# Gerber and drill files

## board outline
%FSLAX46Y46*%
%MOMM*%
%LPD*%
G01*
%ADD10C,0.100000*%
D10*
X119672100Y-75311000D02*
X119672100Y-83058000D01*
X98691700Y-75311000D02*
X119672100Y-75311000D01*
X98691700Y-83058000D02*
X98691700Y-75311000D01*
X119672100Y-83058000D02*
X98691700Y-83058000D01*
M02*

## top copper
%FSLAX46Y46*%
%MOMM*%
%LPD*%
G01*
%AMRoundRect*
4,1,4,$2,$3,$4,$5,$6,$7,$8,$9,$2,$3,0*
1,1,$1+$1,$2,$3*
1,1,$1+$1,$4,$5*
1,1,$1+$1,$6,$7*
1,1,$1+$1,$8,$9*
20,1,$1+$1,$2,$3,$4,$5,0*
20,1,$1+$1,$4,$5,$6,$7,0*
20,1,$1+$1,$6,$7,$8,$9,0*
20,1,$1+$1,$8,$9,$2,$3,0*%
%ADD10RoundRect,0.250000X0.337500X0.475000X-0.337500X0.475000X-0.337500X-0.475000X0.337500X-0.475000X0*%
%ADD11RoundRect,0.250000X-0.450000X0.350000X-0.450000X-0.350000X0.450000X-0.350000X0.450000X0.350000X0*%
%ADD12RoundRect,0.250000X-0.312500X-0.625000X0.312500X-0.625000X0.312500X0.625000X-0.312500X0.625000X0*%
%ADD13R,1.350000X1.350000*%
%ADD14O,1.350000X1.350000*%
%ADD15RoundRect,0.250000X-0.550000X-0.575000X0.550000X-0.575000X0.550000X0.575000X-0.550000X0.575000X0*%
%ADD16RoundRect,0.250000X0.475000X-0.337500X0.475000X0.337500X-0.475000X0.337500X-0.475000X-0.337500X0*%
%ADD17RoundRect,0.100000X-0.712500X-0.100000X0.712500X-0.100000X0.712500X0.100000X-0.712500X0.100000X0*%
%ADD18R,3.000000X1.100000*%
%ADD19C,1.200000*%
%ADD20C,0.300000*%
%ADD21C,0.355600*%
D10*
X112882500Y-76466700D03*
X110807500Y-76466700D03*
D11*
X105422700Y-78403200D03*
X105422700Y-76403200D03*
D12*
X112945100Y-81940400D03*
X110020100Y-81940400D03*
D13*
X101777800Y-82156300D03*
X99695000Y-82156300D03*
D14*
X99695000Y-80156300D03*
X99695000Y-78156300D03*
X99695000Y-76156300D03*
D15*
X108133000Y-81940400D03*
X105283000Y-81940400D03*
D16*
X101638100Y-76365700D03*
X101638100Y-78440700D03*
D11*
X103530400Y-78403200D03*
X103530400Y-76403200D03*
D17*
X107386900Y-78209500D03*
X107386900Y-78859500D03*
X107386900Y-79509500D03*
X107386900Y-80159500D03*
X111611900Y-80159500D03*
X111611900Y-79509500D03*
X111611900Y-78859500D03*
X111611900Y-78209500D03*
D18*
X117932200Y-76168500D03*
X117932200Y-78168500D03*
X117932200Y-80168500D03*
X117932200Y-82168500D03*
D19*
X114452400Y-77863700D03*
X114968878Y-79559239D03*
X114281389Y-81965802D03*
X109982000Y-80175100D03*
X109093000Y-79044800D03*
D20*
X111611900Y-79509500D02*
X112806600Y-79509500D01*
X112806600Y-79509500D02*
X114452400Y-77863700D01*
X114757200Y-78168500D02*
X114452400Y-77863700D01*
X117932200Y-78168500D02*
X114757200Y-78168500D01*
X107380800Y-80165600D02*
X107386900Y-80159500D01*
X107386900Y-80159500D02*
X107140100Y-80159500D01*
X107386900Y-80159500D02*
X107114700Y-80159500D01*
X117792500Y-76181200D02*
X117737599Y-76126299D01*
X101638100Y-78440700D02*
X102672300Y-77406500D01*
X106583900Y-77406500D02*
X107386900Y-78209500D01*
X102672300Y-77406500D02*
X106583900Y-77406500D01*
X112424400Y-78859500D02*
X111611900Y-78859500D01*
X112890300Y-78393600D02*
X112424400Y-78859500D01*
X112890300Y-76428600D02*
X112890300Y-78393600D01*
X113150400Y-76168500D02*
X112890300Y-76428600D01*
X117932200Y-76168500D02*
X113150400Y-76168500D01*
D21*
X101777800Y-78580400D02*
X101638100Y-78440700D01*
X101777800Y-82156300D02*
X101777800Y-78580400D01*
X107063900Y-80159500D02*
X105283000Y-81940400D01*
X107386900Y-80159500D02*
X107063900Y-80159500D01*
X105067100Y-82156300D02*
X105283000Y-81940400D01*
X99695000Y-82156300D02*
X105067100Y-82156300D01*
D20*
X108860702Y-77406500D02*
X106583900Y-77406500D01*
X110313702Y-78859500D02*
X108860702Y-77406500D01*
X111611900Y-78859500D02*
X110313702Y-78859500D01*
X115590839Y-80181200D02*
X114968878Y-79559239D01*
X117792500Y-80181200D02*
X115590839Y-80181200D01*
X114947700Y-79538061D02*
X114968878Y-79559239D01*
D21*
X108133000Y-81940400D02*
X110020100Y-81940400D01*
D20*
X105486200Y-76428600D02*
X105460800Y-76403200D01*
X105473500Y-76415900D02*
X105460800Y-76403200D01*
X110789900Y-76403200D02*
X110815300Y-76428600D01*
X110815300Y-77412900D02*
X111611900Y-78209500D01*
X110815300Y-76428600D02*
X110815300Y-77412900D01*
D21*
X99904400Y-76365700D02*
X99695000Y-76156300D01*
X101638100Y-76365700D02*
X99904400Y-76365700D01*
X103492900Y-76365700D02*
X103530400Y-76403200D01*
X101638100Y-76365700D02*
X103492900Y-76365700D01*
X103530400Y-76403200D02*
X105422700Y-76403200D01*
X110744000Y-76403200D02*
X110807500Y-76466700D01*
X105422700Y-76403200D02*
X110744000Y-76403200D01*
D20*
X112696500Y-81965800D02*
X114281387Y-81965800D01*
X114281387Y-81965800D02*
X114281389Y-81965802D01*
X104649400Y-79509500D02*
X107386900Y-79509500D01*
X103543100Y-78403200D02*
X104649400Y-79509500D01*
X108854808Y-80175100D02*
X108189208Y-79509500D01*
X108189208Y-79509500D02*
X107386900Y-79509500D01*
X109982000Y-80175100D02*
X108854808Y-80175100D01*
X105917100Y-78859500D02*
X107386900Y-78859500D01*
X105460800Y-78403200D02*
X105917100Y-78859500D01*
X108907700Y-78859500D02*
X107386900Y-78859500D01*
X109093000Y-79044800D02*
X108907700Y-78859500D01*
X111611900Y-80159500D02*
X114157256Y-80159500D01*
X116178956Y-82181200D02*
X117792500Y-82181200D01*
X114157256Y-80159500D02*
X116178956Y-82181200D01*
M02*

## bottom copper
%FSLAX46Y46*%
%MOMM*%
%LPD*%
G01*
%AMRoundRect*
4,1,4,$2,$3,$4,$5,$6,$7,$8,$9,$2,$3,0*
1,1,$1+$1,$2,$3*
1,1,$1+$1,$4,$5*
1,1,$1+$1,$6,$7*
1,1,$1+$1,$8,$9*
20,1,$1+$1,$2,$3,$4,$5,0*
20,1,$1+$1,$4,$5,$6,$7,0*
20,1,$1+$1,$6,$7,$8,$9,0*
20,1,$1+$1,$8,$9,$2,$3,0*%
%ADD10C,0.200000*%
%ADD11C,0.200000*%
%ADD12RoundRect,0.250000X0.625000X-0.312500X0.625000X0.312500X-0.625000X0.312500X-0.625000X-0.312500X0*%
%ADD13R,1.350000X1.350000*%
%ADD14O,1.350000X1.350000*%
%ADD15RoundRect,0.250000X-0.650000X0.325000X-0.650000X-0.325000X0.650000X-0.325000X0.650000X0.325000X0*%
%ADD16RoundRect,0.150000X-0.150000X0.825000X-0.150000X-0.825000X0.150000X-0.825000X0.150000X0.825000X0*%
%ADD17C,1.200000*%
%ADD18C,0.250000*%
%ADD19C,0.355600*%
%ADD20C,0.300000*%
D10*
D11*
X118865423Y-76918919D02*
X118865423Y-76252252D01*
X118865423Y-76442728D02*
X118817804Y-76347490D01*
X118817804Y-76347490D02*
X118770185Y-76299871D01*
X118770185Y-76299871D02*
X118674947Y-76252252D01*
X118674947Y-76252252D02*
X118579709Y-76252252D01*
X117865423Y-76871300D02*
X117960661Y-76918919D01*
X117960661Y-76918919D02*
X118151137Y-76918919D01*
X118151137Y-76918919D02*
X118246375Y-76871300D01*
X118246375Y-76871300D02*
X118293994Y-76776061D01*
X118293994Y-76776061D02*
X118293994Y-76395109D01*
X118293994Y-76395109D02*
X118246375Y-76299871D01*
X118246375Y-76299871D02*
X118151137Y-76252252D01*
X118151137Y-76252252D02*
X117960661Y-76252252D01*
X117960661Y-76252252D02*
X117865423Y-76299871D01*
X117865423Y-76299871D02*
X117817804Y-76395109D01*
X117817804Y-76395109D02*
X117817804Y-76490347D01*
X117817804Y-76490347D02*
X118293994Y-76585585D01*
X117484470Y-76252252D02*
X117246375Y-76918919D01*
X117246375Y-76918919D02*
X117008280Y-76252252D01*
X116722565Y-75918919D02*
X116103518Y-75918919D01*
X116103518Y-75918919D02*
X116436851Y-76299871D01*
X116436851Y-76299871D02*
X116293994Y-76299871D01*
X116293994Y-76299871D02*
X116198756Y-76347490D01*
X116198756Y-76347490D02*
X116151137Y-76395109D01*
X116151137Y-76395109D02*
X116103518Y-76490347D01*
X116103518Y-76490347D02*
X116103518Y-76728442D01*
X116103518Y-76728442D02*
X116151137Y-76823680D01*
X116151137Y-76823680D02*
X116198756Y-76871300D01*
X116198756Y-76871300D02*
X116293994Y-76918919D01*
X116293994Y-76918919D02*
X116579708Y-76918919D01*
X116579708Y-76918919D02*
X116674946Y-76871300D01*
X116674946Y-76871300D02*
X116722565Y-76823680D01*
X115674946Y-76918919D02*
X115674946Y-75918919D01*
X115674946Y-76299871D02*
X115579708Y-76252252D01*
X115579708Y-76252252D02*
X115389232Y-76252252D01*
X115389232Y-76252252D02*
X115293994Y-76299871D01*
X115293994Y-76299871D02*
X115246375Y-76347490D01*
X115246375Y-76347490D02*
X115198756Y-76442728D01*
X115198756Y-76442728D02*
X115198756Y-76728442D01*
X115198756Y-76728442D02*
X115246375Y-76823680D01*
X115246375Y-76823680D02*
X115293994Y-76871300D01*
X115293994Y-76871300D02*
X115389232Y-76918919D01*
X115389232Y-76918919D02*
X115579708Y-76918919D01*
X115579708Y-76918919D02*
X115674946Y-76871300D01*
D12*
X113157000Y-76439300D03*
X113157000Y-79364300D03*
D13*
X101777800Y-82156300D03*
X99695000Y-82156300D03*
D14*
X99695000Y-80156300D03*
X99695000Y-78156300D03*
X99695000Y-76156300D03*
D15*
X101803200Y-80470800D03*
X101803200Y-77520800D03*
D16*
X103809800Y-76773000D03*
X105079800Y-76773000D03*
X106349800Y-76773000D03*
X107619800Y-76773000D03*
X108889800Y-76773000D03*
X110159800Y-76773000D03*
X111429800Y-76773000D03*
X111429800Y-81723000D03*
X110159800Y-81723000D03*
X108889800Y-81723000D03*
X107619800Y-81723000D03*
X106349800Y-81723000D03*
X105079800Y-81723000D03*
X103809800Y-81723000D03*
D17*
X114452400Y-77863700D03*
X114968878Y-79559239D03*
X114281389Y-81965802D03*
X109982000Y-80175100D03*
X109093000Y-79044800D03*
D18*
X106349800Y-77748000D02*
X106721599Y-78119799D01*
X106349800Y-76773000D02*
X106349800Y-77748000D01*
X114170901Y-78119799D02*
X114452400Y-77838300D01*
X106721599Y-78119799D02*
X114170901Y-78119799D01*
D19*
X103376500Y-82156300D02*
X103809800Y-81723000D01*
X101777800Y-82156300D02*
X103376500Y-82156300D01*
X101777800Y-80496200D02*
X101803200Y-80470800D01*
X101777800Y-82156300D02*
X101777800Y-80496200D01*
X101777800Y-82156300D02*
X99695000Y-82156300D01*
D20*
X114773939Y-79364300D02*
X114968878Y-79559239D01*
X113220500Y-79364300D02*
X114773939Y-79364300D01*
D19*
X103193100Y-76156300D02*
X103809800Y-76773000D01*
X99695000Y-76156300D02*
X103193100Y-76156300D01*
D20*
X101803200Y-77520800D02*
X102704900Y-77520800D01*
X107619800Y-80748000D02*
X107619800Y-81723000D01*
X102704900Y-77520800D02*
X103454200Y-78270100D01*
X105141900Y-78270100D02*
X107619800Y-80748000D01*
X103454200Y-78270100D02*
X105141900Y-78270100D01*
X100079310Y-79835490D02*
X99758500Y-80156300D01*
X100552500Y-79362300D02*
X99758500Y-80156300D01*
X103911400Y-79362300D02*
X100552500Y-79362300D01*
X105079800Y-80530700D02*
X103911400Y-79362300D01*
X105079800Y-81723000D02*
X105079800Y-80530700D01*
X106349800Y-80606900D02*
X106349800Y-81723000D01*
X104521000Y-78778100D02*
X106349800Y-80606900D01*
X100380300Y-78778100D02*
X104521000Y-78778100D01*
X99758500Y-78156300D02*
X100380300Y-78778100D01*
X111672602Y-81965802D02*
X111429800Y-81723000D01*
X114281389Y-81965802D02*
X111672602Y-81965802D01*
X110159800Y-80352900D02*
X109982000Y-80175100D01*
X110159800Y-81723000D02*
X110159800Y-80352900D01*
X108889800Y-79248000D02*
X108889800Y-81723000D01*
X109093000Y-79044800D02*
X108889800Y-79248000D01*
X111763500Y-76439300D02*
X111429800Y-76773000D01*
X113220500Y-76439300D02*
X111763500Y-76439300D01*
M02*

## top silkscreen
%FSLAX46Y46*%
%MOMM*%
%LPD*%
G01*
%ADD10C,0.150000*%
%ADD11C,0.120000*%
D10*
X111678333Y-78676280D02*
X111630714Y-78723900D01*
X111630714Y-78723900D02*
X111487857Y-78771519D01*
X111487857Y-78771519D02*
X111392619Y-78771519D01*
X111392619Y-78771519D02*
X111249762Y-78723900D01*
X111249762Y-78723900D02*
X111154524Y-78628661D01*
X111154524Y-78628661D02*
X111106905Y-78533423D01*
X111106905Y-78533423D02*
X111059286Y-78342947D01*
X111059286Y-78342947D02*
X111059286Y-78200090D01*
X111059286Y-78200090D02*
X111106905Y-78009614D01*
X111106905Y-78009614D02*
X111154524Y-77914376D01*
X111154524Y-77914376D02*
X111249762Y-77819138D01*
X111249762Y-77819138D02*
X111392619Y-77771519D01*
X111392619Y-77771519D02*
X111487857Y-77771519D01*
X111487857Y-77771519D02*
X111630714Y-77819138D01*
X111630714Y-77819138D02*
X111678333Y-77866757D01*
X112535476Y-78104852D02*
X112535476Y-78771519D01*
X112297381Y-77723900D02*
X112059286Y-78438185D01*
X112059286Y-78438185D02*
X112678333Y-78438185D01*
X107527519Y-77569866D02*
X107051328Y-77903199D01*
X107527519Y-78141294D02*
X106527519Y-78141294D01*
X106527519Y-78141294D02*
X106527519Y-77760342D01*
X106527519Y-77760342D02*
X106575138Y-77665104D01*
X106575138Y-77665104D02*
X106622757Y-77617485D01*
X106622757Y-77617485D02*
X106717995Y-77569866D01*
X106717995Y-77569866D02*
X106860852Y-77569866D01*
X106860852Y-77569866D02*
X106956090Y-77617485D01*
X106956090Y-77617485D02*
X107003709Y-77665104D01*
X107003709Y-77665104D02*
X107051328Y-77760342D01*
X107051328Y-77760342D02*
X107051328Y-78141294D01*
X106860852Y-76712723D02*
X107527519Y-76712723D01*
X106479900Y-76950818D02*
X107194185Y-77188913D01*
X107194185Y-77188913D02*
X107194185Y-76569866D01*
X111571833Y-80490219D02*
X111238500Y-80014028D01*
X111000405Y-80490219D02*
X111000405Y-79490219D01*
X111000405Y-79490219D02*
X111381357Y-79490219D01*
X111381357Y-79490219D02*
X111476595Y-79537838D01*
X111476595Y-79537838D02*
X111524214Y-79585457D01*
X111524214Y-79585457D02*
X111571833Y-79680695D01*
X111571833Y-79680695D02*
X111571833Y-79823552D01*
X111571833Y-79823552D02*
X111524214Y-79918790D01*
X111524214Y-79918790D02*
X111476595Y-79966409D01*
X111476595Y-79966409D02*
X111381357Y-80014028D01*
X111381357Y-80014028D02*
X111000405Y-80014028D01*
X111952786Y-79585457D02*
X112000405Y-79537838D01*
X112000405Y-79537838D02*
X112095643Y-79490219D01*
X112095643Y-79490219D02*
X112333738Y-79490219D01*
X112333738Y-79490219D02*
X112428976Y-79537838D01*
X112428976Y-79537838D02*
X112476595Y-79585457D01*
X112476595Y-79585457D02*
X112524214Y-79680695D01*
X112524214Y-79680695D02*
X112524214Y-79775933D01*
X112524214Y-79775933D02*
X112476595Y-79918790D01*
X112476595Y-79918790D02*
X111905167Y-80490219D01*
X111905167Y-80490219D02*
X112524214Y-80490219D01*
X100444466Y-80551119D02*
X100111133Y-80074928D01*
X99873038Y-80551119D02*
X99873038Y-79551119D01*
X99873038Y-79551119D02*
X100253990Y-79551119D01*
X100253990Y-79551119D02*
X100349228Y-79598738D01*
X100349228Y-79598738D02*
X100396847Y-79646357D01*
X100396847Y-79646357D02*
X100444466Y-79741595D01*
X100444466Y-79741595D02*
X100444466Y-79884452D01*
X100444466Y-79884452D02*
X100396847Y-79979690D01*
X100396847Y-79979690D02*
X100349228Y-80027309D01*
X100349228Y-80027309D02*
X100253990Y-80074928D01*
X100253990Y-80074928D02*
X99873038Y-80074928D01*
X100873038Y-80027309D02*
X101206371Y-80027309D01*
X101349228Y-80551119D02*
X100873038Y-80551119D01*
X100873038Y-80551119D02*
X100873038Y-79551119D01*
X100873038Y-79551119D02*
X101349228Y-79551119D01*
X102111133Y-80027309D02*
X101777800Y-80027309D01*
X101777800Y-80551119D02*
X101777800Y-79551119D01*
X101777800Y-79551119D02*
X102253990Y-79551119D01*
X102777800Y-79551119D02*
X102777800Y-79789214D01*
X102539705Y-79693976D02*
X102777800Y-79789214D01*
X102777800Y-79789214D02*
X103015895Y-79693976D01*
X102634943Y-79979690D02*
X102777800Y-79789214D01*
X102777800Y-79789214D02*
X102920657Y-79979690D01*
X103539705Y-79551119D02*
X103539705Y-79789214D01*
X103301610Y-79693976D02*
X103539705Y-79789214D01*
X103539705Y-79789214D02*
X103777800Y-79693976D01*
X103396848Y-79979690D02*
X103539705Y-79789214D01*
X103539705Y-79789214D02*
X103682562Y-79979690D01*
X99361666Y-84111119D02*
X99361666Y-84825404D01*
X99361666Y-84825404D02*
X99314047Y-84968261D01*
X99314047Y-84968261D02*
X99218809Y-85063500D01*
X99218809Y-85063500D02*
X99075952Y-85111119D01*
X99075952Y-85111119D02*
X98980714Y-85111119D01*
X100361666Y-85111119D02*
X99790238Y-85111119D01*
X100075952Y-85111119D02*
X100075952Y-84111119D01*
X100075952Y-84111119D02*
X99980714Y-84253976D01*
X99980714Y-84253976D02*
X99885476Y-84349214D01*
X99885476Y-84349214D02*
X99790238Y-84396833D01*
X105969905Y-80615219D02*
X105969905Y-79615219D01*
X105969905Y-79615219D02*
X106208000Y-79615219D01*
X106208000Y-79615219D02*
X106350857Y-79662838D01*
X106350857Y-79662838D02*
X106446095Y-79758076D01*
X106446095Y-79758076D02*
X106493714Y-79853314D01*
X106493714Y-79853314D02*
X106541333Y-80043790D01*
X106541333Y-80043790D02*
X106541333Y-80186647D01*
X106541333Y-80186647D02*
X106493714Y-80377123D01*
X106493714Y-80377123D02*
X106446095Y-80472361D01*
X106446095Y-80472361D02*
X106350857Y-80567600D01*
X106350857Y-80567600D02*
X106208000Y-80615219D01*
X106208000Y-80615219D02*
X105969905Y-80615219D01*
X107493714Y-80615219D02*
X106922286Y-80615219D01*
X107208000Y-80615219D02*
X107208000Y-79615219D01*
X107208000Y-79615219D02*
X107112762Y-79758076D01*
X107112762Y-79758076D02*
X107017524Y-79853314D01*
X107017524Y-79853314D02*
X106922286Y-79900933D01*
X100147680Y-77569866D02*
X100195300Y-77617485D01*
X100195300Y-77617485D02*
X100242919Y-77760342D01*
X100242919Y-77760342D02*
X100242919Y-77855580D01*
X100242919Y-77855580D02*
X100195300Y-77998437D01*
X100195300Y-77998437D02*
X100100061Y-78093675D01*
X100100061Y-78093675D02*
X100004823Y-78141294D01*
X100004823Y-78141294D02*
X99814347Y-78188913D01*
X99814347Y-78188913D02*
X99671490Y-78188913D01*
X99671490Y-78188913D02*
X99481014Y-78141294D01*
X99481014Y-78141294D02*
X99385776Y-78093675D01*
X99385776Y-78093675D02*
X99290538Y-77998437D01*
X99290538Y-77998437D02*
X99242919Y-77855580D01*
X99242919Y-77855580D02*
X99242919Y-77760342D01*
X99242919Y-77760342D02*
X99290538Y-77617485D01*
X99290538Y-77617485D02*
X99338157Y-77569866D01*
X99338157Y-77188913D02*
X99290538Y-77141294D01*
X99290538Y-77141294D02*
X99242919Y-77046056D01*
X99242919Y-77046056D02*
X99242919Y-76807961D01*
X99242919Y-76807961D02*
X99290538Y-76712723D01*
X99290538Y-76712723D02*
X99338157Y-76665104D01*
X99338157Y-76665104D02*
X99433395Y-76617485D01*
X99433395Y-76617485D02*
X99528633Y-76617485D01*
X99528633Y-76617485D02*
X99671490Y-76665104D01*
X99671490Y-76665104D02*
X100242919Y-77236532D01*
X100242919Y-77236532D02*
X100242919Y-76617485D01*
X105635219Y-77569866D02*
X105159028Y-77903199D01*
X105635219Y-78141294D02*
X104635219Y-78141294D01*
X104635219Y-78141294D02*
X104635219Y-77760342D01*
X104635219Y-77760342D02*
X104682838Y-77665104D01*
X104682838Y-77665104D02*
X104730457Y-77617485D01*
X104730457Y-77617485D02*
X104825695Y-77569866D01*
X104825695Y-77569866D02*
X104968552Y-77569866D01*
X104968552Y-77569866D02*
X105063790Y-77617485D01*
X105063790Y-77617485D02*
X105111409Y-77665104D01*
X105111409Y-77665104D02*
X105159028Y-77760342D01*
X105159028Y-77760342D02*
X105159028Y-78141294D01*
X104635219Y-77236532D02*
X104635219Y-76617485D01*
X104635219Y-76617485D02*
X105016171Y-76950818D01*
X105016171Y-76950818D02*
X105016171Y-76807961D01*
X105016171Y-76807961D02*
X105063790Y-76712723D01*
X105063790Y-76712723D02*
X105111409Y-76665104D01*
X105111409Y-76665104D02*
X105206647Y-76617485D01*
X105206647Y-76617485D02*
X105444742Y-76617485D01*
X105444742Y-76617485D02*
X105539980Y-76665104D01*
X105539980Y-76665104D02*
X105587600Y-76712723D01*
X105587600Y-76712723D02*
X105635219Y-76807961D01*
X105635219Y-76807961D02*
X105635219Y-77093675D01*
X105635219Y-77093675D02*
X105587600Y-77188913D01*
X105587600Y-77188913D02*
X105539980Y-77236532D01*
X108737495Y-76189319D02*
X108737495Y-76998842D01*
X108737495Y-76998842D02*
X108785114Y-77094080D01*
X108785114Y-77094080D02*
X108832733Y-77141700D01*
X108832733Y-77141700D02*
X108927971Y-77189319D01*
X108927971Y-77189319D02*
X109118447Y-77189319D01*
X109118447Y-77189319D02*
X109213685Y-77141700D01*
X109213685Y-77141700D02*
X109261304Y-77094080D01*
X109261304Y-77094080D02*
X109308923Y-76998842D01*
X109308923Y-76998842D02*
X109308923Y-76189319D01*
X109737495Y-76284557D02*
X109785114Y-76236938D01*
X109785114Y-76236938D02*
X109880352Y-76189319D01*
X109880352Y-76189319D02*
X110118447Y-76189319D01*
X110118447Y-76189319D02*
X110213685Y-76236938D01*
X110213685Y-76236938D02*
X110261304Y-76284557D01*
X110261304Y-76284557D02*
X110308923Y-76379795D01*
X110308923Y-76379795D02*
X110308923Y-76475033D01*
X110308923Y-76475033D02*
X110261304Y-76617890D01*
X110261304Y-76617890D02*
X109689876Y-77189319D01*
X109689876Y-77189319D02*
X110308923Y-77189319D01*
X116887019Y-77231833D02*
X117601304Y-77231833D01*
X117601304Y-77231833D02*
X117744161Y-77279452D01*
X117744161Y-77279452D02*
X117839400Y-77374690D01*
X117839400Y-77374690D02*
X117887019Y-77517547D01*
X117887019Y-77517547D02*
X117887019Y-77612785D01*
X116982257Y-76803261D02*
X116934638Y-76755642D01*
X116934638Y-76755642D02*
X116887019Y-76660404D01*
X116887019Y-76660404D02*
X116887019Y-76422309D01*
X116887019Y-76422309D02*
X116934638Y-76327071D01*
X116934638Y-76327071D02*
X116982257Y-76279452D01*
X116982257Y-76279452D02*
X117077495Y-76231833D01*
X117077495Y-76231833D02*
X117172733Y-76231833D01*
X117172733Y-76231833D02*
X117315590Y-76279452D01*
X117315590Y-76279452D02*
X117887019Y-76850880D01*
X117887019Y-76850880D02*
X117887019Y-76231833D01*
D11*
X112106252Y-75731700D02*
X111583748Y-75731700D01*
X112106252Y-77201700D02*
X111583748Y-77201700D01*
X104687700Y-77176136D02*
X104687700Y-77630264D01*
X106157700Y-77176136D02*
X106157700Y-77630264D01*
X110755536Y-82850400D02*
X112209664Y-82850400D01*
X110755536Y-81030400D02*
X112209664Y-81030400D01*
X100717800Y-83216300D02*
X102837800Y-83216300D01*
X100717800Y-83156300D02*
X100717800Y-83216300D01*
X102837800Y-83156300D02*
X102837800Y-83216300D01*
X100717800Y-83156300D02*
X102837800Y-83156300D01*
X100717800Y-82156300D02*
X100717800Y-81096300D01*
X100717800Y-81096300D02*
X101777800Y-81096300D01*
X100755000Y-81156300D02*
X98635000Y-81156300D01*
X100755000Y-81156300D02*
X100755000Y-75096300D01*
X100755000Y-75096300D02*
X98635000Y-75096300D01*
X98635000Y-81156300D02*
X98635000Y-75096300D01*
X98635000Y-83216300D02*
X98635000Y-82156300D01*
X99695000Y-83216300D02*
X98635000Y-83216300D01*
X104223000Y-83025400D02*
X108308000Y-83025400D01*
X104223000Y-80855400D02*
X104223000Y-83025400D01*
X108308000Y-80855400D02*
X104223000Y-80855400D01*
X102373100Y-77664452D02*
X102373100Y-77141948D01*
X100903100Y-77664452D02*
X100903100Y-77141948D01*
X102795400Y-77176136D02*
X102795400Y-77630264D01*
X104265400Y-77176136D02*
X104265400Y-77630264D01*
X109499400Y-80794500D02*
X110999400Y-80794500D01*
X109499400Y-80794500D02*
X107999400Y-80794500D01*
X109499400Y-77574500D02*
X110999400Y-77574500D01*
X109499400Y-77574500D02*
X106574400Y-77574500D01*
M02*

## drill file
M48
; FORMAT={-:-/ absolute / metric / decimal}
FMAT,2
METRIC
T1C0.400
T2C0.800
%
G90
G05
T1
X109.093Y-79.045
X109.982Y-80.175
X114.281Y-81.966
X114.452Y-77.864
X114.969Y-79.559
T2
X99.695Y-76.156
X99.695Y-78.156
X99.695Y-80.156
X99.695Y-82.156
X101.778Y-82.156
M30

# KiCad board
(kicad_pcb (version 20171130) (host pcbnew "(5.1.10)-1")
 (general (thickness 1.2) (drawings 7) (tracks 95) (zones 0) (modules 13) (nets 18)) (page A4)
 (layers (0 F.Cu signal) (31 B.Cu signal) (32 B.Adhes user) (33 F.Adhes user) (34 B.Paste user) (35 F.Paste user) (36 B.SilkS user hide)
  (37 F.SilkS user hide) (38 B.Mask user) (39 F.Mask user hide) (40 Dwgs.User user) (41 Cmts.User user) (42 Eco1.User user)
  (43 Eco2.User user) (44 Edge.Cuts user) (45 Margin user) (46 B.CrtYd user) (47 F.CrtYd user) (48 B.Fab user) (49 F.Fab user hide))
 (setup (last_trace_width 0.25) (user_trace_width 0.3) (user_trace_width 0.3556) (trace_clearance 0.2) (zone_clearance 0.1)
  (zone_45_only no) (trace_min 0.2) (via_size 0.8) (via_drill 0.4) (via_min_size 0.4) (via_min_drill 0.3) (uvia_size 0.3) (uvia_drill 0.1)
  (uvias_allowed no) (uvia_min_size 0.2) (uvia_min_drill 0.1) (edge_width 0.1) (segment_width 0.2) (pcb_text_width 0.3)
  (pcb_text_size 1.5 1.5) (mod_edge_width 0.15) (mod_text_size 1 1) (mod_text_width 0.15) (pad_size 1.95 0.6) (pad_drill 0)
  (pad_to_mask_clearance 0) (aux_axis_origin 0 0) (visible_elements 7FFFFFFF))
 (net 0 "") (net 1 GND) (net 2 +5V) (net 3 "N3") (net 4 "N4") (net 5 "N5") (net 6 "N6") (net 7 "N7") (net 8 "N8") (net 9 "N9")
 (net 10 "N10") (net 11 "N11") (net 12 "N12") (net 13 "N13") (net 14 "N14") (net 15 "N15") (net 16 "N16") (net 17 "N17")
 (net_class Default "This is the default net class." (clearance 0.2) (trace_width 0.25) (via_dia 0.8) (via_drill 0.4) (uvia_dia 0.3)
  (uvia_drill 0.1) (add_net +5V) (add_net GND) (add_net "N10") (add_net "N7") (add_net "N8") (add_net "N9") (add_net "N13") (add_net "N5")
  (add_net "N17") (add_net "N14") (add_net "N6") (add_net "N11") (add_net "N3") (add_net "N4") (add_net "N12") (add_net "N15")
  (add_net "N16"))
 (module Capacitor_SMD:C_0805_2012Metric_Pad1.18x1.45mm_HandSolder (layer F.Cu) (at 111.845 76.4667 180)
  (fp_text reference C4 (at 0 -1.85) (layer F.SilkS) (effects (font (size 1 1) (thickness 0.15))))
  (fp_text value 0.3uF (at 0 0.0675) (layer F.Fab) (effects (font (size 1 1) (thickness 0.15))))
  (fp_line (start -0.261252 0.735) (end 0.261252 0.735) (layer F.SilkS) (width 0.12))
  (fp_line (start -0.261252 -0.735) (end 0.261252 -0.735) (layer F.SilkS) (width 0.12))
  (pad 1 smd roundrect (at -1.0375 0 180) (size 1.175 1.45) (layers F.Cu F.Paste F.Mask) (roundrect_rratio 0.212766) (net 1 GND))
  (pad 2 smd roundrect (at 1.0375 0 180) (size 1.175 1.45) (layers F.Cu F.Paste F.Mask) (roundrect_rratio 0.212766) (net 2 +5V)))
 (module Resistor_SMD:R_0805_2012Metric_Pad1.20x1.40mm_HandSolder (layer F.Cu) (at 105.4227 77.4032 270)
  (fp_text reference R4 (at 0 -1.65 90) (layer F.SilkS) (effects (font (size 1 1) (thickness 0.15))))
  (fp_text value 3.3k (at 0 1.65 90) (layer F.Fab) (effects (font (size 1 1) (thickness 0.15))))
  (fp_line (start -0.227064 0.735) (end 0.227064 0.735) (layer F.SilkS) (width 0.12))
  (fp_line (start -0.227064 -0.735) (end 0.227064 -0.735) (layer F.SilkS) (width 0.12))
  (pad 2 smd roundrect (at 1 0 270) (size 1.2 1.4) (layers F.Cu F.Paste F.Mask) (roundrect_rratio 0.208333) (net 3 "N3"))
  (pad 1 smd roundrect (at -1 0 270) (size 1.2 1.4) (layers F.Cu F.Paste F.Mask) (roundrect_rratio 0.208333) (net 2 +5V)))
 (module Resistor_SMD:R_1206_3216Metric (layer B.Cu) (at 113.157 77.9018 90)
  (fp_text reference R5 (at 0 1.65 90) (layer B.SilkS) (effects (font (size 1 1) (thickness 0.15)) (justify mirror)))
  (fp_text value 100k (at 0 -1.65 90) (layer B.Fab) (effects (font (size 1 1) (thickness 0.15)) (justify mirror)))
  (pad 2 smd roundrect (at 1.4625 0 90) (size 1.125 1.75) (layers B.Cu B.Paste B.Mask) (roundrect_rratio 0.222222) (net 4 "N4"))
  (pad 1 smd roundrect (at -1.4625 0 90) (size 1.125 1.75) (layers B.Cu B.Paste B.Mask) (roundrect_rratio 0.222222) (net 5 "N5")))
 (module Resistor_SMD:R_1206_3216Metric (layer F.Cu) (at 111.4826 81.9404)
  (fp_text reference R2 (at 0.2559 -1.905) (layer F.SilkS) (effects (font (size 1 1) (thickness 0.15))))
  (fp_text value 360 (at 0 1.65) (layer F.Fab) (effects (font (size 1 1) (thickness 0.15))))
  (fp_line (start -0.727064 0.91) (end 0.727064 0.91) (layer F.SilkS) (width 0.12))
  (fp_line (start -0.727064 -0.91) (end 0.727064 -0.91) (layer F.SilkS) (width 0.12))
  (pad 2 smd roundrect (at 1.4625 0) (size 1.125 1.75) (layers F.Cu F.Paste F.Mask) (roundrect_rratio 0.222222) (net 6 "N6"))
  (pad 1 smd roundrect (at -1.4625 0) (size 1.125 1.75) (layers F.Cu F.Paste F.Mask) (roundrect_rratio 0.222222) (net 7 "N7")))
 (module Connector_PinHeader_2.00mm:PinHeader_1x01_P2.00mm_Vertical (layer F.Cu) (at 101.7778 82.1563)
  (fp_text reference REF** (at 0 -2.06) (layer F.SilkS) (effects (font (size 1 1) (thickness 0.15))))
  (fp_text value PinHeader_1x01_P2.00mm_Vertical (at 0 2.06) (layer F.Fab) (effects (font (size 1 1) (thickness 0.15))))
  (fp_line (start -1.06 1.06) (end 1.06 1.06) (layer F.SilkS) (width 0.12))
  (fp_line (start -1.06 1) (end -1.06 1.06) (layer F.SilkS) (width 0.12))
  (fp_line (start 1.06 1) (end 1.06 1.06) (layer F.SilkS) (width 0.12))
  (fp_line (start -1.06 1) (end 1.06 1) (layer F.SilkS) (width 0.12))
  (fp_line (start -1.06 0) (end -1.06 -1.06) (layer F.SilkS) (width 0.12))
  (fp_line (start -1.06 -1.06) (end 0 -1.06) (layer F.SilkS) (width 0.12))
  (pad 1 thru_hole rect (at 0 0) (size 1.35 1.35) (drill 0.8) (layers *.Cu *.Mask) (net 1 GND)))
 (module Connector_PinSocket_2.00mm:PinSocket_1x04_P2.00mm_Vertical (layer F.Cu) (at 99.695 82.1563 180)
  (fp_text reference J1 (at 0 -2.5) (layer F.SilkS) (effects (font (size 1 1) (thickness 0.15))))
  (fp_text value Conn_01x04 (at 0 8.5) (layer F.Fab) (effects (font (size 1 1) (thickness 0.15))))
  (fp_line (start -1.06 1) (end 1.06 1) (layer F.SilkS) (width 0.12))
  (fp_line (start -1.06 1) (end -1.06 7.06) (layer F.SilkS) (width 0.12))
  (fp_line (start -1.06 7.06) (end 1.06 7.06) (layer F.SilkS) (width 0.12))
  (fp_line (start 1.06 1) (end 1.06 7.06) (layer F.SilkS) (width 0.12))
  (fp_line (start 1.06 -1.06) (end 1.06 0) (layer F.SilkS) (width 0.12))
  (fp_line (start 0 -1.06) (end 1.06 -1.06) (layer F.SilkS) (width 0.12))
  (pad 1 thru_hole rect (at 0 0 180) (size 1.35 1.35) (drill 0.8) (layers *.Cu *.Mask) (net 1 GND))
  (pad 2 thru_hole oval (at 0 2 180) (size 1.35 1.35) (drill 0.8) (layers *.Cu *.Mask) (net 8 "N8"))
  (pad 3 thru_hole oval (at 0 4 180) (size 1.35 1.35) (drill 0.8) (layers *.Cu *.Mask) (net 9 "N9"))
  (pad 4 thru_hole oval (at 0 6 180) (size 1.35 1.35) (drill 0.8) (layers *.Cu *.Mask) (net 2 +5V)))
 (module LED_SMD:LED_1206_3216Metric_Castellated (layer F.Cu) (at 106.708 81.9404)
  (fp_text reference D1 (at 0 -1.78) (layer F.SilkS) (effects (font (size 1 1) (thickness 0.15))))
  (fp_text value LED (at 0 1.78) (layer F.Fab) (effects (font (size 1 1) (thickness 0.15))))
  (fp_line (start -2.485 1.085) (end 1.6 1.085) (layer F.SilkS) (width 0.12))
  (fp_line (start -2.485 -1.085) (end -2.485 1.085) (layer F.SilkS) (width 0.12))
  (fp_line (start 1.6 -1.085) (end -2.485 -1.085) (layer F.SilkS) (width 0.12))
  (pad 2 smd roundrect (at 1.425 0) (size 1.6 1.65) (layers F.Cu F.Paste F.Mask) (roundrect_rratio 0.15625) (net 7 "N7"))
  (pad 1 smd roundrect (at -1.425 0) (size 1.6 1.65) (layers F.Cu F.Paste F.Mask) (roundrect_rratio 0.15625) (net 1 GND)))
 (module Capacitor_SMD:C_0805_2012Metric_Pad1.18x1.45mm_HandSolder (layer F.Cu) (at 101.6381 77.4032 90)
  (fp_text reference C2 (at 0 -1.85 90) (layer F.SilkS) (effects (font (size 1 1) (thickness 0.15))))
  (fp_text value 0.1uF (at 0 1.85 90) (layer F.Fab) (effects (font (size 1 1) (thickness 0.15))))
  (fp_line (start -0.261252 0.735) (end 0.261252 0.735) (layer F.SilkS) (width 0.12))
  (fp_line (start -0.261252 -0.735) (end 0.261252 -0.735) (layer F.SilkS) (width 0.12))
  (pad 2 smd roundrect (at 1.0375 0 90) (size 1.175 1.45) (layers F.Cu F.Paste F.Mask) (roundrect_rratio 0.212766) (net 2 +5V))
  (pad 1 smd roundrect (at -1.0375 0 90) (size 1.175 1.45) (layers F.Cu F.Paste F.Mask) (roundrect_rratio 0.212766) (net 1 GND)))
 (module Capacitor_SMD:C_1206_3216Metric (layer B.Cu) (at 101.8032 78.9958 270)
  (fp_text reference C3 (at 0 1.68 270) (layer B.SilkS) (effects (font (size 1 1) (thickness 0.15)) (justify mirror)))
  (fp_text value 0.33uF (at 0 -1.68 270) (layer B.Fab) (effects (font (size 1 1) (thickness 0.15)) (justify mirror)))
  (pad 2 smd roundrect (at 1.475 0 270) (size 1.15 1.8) (layers B.Cu B.Paste B.Mask) (roundrect_rratio 0.217391) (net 1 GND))
  (pad 1 smd roundrect (at -1.475 0 270) (size 1.15 1.8) (layers B.Cu B.Paste B.Mask) (roundrect_rratio 0.217391) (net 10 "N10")))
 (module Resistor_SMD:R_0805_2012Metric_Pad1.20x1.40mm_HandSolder (layer F.Cu) (at 103.5304 77.4032 270)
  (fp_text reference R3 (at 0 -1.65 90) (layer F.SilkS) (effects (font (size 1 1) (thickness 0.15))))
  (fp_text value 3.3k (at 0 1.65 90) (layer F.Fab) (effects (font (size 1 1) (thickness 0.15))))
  (fp_line (start -0.227064 0.735) (end 0.227064 0.735) (layer F.SilkS) (width 0.12))
  (fp_line (start -0.227064 -0.735) (end 0.227064 -0.735) (layer F.SilkS) (width 0.12))
  (pad 2 smd roundrect (at 1 0 270) (size 1.2 1.4) (layers F.Cu F.Paste F.Mask) (roundrect_rratio 0.208333) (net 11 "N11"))
  (pad 1 smd roundrect (at -1 0 270) (size 1.2 1.4) (layers F.Cu F.Paste F.Mask) (roundrect_rratio 0.208333) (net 2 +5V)))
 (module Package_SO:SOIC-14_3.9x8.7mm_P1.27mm (layer B.Cu) (at 107.6198 79.248 270)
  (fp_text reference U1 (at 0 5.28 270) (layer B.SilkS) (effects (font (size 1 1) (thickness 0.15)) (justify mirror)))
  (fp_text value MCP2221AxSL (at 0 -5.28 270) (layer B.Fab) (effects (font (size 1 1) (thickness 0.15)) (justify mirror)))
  (pad 1 smd roundrect (at -2.475 3.81 270) (size 1.95 0.6) (layers B.Cu B.Paste B.Mask) (roundrect_rratio 0.25) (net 2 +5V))
  (pad 2 smd roundrect (at -2.475 2.54 270) (size 1.95 0.6) (layers B.Cu B.Paste B.Mask) (roundrect_rratio 0.25) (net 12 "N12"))
  (pad 3 smd roundrect (at -2.475 1.27 270) (size 1.95 0.6) (layers B.Cu B.Paste B.Mask) (roundrect_rratio 0.25) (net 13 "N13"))
  (pad 4 smd roundrect (at -2.475 0 270) (size 1.95 0.6) (layers B.Cu B.Paste B.Mask) (roundrect_rratio 0.25) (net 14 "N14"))
  (pad 5 smd roundrect (at -2.475 -1.27 270) (size 1.95 0.6) (layers B.Cu B.Paste B.Mask) (roundrect_rratio 0.25) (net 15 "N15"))
  (pad 6 smd roundrect (at -2.475 -2.54 270) (size 1.95 0.6) (layers B.Cu B.Paste B.Mask) (roundrect_rratio 0.25) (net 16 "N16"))
  (pad 7 smd roundrect (at -2.475 -3.81 270) (size 1.95 0.6) (layers B.Cu B.Paste B.Mask) (roundrect_rratio 0.25) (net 4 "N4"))
  (pad 8 smd roundrect (at 2.475 -3.81 270) (size 1.95 0.6) (layers B.Cu B.Paste B.Mask) (roundrect_rratio 0.25) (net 6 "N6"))
  (pad 9 smd roundrect (at 2.475 -2.54 270) (size 1.95 0.6) (layers B.Cu B.Paste B.Mask) (roundrect_rratio 0.25) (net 11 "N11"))
  (pad 10 smd roundrect (at 2.475 -1.27 270) (size 1.95 0.6) (layers B.Cu B.Paste B.Mask) (roundrect_rratio 0.25) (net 3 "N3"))
  (pad 11 smd roundrect (at 2.475 0 270) (size 1.95 0.6) (layers B.Cu B.Paste B.Mask) (roundrect_rratio 0.25) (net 10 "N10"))
  (pad 12 smd roundrect (at 2.475 1.27 270) (size 1.95 0.6) (layers B.Cu B.Paste B.Mask) (roundrect_rratio 0.25) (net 9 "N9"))
  (pad 13 smd roundrect (at 2.475 2.54 270) (size 1.95 0.6) (layers B.Cu B.Paste B.Mask) (roundrect_rratio 0.25) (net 8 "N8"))
  (pad 14 smd roundrect (at 2.475 3.81 270) (size 1.95 0.6) (layers B.Cu B.Paste B.Mask) (roundrect_rratio 0.25) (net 1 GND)))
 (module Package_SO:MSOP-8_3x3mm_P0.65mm (layer F.Cu) (at 109.4994 79.1845)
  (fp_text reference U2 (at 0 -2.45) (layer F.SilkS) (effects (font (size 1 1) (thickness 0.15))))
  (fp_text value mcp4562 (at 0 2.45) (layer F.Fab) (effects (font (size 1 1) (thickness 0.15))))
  (fp_line (start 0 1.61) (end 1.5 1.61) (layer F.SilkS) (width 0.12))
  (fp_line (start 0 1.61) (end -1.5 1.61) (layer F.SilkS) (width 0.12))
  (fp_line (start 0 -1.61) (end 1.5 -1.61) (layer F.SilkS) (width 0.12))
  (fp_line (start 0 -1.61) (end -2.925 -1.61) (layer F.SilkS) (width 0.12))
  (pad 1 smd roundrect (at -2.1125 -0.975) (size 1.625 0.4) (layers F.Cu F.Paste F.Mask) (roundrect_rratio 0.25) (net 1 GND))
  (pad 2 smd roundrect (at -2.1125 -0.325) (size 1.625 0.4) (layers F.Cu F.Paste F.Mask) (roundrect_rratio 0.25) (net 3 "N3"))
  (pad 3 smd roundrect (at -2.1125 0.325) (size 1.625 0.4) (layers F.Cu F.Paste F.Mask) (roundrect_rratio 0.25) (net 11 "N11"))
  (pad 4 smd roundrect (at -2.1125 0.975) (size 1.625 0.4) (layers F.Cu F.Paste F.Mask) (roundrect_rratio 0.25) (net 1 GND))
  (pad 5 smd roundrect (at 2.1125 0.975) (size 1.625 0.4) (layers F.Cu F.Paste F.Mask) (roundrect_rratio 0.25) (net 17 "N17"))
  (pad 6 smd roundrect (at 2.1125 0.325) (size 1.625 0.4) (layers F.Cu F.Paste F.Mask) (roundrect_rratio 0.25) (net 13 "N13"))
  (pad 7 smd roundrect (at 2.1125 -0.325) (size 1.625 0.4) (layers F.Cu F.Paste F.Mask) (roundrect_rratio 0.25) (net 1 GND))
  (pad 8 smd roundrect (at 2.1125 -0.975) (size 1.625 0.4) (layers F.Cu F.Paste F.Mask) (roundrect_rratio 0.25) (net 2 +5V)))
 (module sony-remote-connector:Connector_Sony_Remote (layer F.Cu) (at 116.6622 78.1685 270)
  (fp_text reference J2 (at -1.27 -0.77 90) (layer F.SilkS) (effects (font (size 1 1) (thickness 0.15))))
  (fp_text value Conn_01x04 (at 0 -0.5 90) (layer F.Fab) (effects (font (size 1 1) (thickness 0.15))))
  (pad 1 smd rect (at -2 -1.27 270) (size 1.1 3) (layers F.Cu F.Mask) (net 1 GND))
  (pad 2 smd rect (at 0 -1.27 270) (size 1.1 3) (layers F.Cu F.Mask) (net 13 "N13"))
  (pad 3 smd rect (at 2 -1.27 270) (size 1.1 3) (layers F.Cu F.Mask) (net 5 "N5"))
  (pad 4 smd rect (at 4 -1.27 270) (size 1.1 3) (layers F.Cu F.Mask) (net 17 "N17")))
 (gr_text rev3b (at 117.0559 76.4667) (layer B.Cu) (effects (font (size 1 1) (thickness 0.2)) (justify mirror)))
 (gr_line (start 119.6721 75.311) (end 119.6721 83.058) (layer Edge.Cuts) (width 0.1))
 (gr_line (start 98.6917 75.311) (end 119.6721 75.311) (layer Edge.Cuts) (width 0.1))
 (gr_line (start 98.6917 83.058) (end 98.6917 75.311) (layer Edge.Cuts) (width 0.1))
 (gr_line (start 119.6721 83.058) (end 98.6917 83.058) (layer Edge.Cuts) (width 0.1))
 (segment (start 111.6119 79.5095) (end 112.8066 79.5095) (width 0.3) (layer F.Cu) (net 13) (status 10))
 (via (at 114.4524 77.8637) (size 1.2) (drill 0.4) (layers F.Cu B.Cu) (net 13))
 (segment (start 106.3498 77.748) (end 106.721599 78.119799) (width 0.25) (layer B.Cu) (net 13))
 (segment (start 106.3498 76.773) (end 106.3498 77.748) (width 0.25) (layer B.Cu) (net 13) (status 10))
 (segment (start 112.8066 79.5095) (end 114.4524 77.8637) (width 0.3) (layer F.Cu) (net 13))
 (segment (start 114.7572 78.1685) (end 114.4524 77.8637) (width 0.3) (layer F.Cu) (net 13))
 (segment (start 117.9322 78.1685) (end 114.7572 78.1685) (width 0.3) (layer F.Cu) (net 13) (status 10))
 (segment (start 114.170901 78.119799) (end 114.4524 77.8383) (width 0.25) (layer B.Cu) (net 13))
 (segment (start 106.721599 78.119799) (end 114.170901 78.119799) (width 0.25) (layer B.Cu) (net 13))
 (segment (start 107.3808 80.1656) (end 107.3869 80.1595) (width 0.3) (layer F.Cu) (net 1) (status 30))
 (segment (start 107.3869 80.1595) (end 107.1401 80.1595) (width 0.3) (layer F.Cu) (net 1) (status 30))
 (segment (start 107.3869 80.1595) (end 107.1147 80.1595) (width 0.3) (layer F.Cu) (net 1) (status 30))
 (segment (start 117.7925 76.1812) (end 117.737599 76.126299) (width 0.3) (layer F.Cu) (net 1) (status 30))
 (segment (start 101.6381 78.4407) (end 102.6723 77.4065) (width 0.3) (layer F.Cu) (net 1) (status 10))
 (segment (start 106.5839 77.4065) (end 107.3869 78.2095) (width 0.3) (layer F.Cu) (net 1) (status 20))
 (segment (start 102.6723 77.4065) (end 106.5839 77.4065) (width 0.3) (layer F.Cu) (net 1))
 (segment (start 112.4244 78.8595) (end 111.6119 78.8595) (width 0.3) (layer F.Cu) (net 1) (status 20))
 (segment (start 112.8903 78.3936) (end 112.4244 78.8595) (width 0.3) (layer F.Cu) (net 1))
 (segment (start 112.8903 76.4286) (end 112.8903 78.3936) (width 0.3) (layer F.Cu) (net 1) (status 10))
 (segment (start 113.1504 76.1685) (end 112.8903 76.4286) (width 0.3) (layer F.Cu) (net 1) (status 30))
 (segment (start 117.9322 76.1685) (end 113.1504 76.1685) (width 0.3) (layer F.Cu) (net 1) (status 30))
 (segment (start 103.3765 82.1563) (end 103.8098 81.723) (width 0.3556) (layer B.Cu) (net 1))
 (segment (start 101.7778 82.1563) (end 103.3765 82.1563) (width 0.3556) (layer B.Cu) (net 1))
 (segment (start 101.7778 80.4962) (end 101.8032 80.4708) (width 0.3556) (layer B.Cu) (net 1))
 (segment (start 101.7778 82.1563) (end 101.7778 80.4962) (width 0.3556) (layer B.Cu) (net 1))
 (segment (start 101.7778 78.5804) (end 101.6381 78.4407) (width 0.3556) (layer F.Cu) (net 1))
 (segment (start 101.7778 82.1563) (end 101.7778 78.5804) (width 0.3556) (layer F.Cu) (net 1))
 (segment (start 107.0639 80.1595) (end 105.283 81.9404) (width 0.3556) (layer F.Cu) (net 1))
 (segment (start 107.3869 80.1595) (end 107.0639 80.1595) (width 0.3556) (layer F.Cu) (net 1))
 (segment (start 101.7778 82.1563) (end 99.695 82.1563) (width 0.3556) (layer B.Cu) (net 1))
 (segment (start 105.0671 82.1563) (end 105.283 81.9404) (width 0.3556) (layer F.Cu) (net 1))
 (segment (start 99.695 82.1563) (end 105.0671 82.1563) (width 0.3556) (layer F.Cu) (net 1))
 (segment (start 108.860702 77.4065) (end 106.5839 77.4065) (width 0.3) (layer F.Cu) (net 1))
 (segment (start 110.313702 78.8595) (end 108.860702 77.4065) (width 0.3) (layer F.Cu) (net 1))
 (segment (start 111.6119 78.8595) (end 110.313702 78.8595) (width 0.3) (layer F.Cu) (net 1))
 (segment (start 115.590839 80.1812) (end 114.968878 79.559239) (width 0.3) (layer F.Cu) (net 5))
 (segment (start 117.7925 80.1812) (end 115.590839 80.1812) (width 0.3) (layer F.Cu) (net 5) (status 10))
 (segment (start 114.773939 79.3643) (end 114.968878 79.559239) (width 0.3) (layer B.Cu) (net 5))
 (segment (start 113.2205 79.3643) (end 114.773939 79.3643) (width 0.3) (layer B.Cu) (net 5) (status 10))
 (segment (start 114.9477 79.538061) (end 114.968878 79.559239) (width 0.3) (layer F.Cu) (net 5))
 (via (at 114.968878 79.559239) (size 1.2) (drill 0.4) (layers F.Cu B.Cu) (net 5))
 (segment (start 108.133 81.9404) (end 110.0201 81.9404) (width 0.3556) (layer F.Cu) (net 7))
 (segment (start 105.4862 76.4286) (end 105.4608 76.4032) (width 0.3) (layer F.Cu) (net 2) (status 30))
 (segment (start 105.4735 76.4159) (end 105.4608 76.4032) (width 0.3) (layer F.Cu) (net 2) (status 30))
 (segment (start 110.7899 76.4032) (end 110.8153 76.4286) (width 0.3) (layer F.Cu) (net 2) (status 30))
 (segment (start 110.8153 77.4129) (end 111.6119 78.2095) (width 0.3) (layer F.Cu) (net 2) (status 20))
 (segment (start 110.8153 76.4286) (end 110.8153 77.4129) (width 0.3) (layer F.Cu) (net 2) (status 10))
 (segment (start 99.9044 76.3657) (end 99.695 76.1563) (width 0.3556) (layer F.Cu) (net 2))
 (segment (start 101.6381 76.3657) (end 99.9044 76.3657) (width 0.3556) (layer F.Cu) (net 2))
 (segment (start 103.4929 76.3657) (end 103.5304 76.4032) (width 0.3556) (layer F.Cu) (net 2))
 (segment (start 101.6381 76.3657) (end 103.4929 76.3657) (width 0.3556) (layer F.Cu) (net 2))
 (segment (start 103.5304 76.4032) (end 105.4227 76.4032) (width 0.3556) (layer F.Cu) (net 2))
 (segment (start 110.744 76.4032) (end 110.8075 76.4667) (width 0.3556) (layer F.Cu) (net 2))
 (segment (start 105.4227 76.4032) (end 110.744 76.4032) (width 0.3556) (layer F.Cu) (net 2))
 (segment (start 103.1931 76.1563) (end 103.8098 76.773) (width 0.3556) (layer B.Cu) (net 2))
 (segment (start 99.695 76.1563) (end 103.1931 76.1563) (width 0.3556) (layer B.Cu) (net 2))
 (segment (start 101.8032 77.5208) (end 102.7049 77.5208) (width 0.3) (layer B.Cu) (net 10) (status 10))
 (segment (start 107.6198 80.748) (end 107.6198 81.723) (width 0.3) (layer B.Cu) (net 10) (status 30))
 (segment (start 102.7049 77.5208) (end 103.4542 78.2701) (width 0.3) (layer B.Cu) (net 10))
 (segment (start 105.1419 78.2701) (end 107.6198 80.748) (width 0.3) (layer B.Cu) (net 10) (status 20))
 (segment (start 103.4542 78.2701) (end 105.1419 78.2701) (width 0.3) (layer B.Cu) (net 10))
 (segment (start 100.07931 79.83549) (end 99.7585 80.1563) (width 0.3) (layer B.Cu) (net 8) (status 30))
 (segment (start 100.5525 79.3623) (end 99.7585 80.1563) (width 0.3) (layer B.Cu) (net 8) (status 20))
 (segment (start 103.9114 79.3623) (end 100.5525 79.3623) (width 0.3) (layer B.Cu) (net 8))
 (segment (start 105.0798 80.5307) (end 103.9114 79.3623) (width 0.3) (layer B.Cu) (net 8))
 (segment (start 105.0798 81.723) (end 105.0798 80.5307) (width 0.3) (layer B.Cu) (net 8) (status 10))
 (segment (start 106.3498 80.6069) (end 106.3498 81.723) (width 0.3) (layer B.Cu) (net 9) (status 20))
 (segment (start 104.521 78.7781) (end 106.3498 80.6069) (width 0.3) (layer B.Cu) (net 9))
 (segment (start 100.3803 78.7781) (end 104.521 78.7781) (width 0.3) (layer B.Cu) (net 9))
 (segment (start 99.7585 78.1563) (end 100.3803 78.7781) (width 0.3) (layer B.Cu) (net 9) (status 10))
 (segment (start 112.6965 81.9658) (end 114.281387 81.9658) (width 0.3) (layer F.Cu) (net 6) (status 10))
 (via (at 114.281389 81.965802) (size 1.2) (drill 0.4) (layers F.Cu B.Cu) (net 6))
 (segment (start 114.281387 81.9658) (end 114.281389 81.965802) (width 0.3) (layer F.Cu) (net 6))
 (segment (start 111.672602 81.965802) (end 111.4298 81.723) (width 0.3) (layer B.Cu) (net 6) (status 30))
 (segment (start 114.281389 81.965802) (end 111.672602 81.965802) (width 0.3) (layer B.Cu) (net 6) (status 20))
 (segment (start 104.6494 79.5095) (end 107.3869 79.5095) (width 0.3) (layer F.Cu) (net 11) (status 20))
 (segment (start 103.5431 78.4032) (end 104.6494 79.5095) (width 0.3) (layer F.Cu) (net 11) (status 10))
 (via (at 109.982 80.1751) (size 1.2) (drill 0.4) (layers F.Cu B.Cu) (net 11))
 (segment (start 110.1598 80.3529) (end 109.982 80.1751) (width 0.3) (layer B.Cu) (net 11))
 (segment (start 110.1598 81.723) (end 110.1598 80.3529) (width 0.3) (layer B.Cu) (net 11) (status 10))
 (segment (start 108.854808 80.1751) (end 108.189208 79.5095) (width 0.3) (layer F.Cu) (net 11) (status 20))
 (segment (start 108.189208 79.5095) (end 107.3869 79.5095) (width 0.3) (layer F.Cu) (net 11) (status 30))
 (segment (start 109.982 80.1751) (end 108.854808 80.1751) (width 0.3) (layer F.Cu) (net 11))
 (segment (start 105.9171 78.8595) (end 107.3869 78.8595) (width 0.3) (layer F.Cu) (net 3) (status 30))
 (segment (start 105.4608 78.4032) (end 105.9171 78.8595) (width 0.3) (layer F.Cu) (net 3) (status 30))
 (segment (start 108.8898 79.248) (end 108.8898 81.723) (width 0.3) (layer B.Cu) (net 3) (status 20))
 (segment (start 109.093 79.0448) (end 108.8898 79.248) (width 0.3) (layer B.Cu) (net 3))
 (segment (start 108.9077 78.8595) (end 107.3869 78.8595) (width 0.3) (layer F.Cu) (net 3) (status 20))
 (segment (start 109.093 79.0448) (end 108.9077 78.8595) (width 0.3) (layer F.Cu) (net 3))
 (via (at 109.093 79.0448) (size 1.2) (drill 0.4) (layers F.Cu B.Cu) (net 3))
 (segment (start 111.7635 76.4393) (end 111.4298 76.773) (width 0.3) (layer B.Cu) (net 4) (status 20))
 (segment (start 113.2205 76.4393) (end 111.7635 76.4393) (width 0.3) (layer B.Cu) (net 4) (status 10))
 (segment (start 111.6119 80.1595) (end 114.157256 80.1595) (width 0.3) (layer F.Cu) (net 17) (status 10))
 (segment (start 116.178956 82.1812) (end 117.7925 82.1812) (width 0.3) (layer F.Cu) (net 17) (status 20))
 (segment (start 114.157256 80.1595) (end 116.178956 82.1812) (width 0.3) (layer F.Cu) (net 17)))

